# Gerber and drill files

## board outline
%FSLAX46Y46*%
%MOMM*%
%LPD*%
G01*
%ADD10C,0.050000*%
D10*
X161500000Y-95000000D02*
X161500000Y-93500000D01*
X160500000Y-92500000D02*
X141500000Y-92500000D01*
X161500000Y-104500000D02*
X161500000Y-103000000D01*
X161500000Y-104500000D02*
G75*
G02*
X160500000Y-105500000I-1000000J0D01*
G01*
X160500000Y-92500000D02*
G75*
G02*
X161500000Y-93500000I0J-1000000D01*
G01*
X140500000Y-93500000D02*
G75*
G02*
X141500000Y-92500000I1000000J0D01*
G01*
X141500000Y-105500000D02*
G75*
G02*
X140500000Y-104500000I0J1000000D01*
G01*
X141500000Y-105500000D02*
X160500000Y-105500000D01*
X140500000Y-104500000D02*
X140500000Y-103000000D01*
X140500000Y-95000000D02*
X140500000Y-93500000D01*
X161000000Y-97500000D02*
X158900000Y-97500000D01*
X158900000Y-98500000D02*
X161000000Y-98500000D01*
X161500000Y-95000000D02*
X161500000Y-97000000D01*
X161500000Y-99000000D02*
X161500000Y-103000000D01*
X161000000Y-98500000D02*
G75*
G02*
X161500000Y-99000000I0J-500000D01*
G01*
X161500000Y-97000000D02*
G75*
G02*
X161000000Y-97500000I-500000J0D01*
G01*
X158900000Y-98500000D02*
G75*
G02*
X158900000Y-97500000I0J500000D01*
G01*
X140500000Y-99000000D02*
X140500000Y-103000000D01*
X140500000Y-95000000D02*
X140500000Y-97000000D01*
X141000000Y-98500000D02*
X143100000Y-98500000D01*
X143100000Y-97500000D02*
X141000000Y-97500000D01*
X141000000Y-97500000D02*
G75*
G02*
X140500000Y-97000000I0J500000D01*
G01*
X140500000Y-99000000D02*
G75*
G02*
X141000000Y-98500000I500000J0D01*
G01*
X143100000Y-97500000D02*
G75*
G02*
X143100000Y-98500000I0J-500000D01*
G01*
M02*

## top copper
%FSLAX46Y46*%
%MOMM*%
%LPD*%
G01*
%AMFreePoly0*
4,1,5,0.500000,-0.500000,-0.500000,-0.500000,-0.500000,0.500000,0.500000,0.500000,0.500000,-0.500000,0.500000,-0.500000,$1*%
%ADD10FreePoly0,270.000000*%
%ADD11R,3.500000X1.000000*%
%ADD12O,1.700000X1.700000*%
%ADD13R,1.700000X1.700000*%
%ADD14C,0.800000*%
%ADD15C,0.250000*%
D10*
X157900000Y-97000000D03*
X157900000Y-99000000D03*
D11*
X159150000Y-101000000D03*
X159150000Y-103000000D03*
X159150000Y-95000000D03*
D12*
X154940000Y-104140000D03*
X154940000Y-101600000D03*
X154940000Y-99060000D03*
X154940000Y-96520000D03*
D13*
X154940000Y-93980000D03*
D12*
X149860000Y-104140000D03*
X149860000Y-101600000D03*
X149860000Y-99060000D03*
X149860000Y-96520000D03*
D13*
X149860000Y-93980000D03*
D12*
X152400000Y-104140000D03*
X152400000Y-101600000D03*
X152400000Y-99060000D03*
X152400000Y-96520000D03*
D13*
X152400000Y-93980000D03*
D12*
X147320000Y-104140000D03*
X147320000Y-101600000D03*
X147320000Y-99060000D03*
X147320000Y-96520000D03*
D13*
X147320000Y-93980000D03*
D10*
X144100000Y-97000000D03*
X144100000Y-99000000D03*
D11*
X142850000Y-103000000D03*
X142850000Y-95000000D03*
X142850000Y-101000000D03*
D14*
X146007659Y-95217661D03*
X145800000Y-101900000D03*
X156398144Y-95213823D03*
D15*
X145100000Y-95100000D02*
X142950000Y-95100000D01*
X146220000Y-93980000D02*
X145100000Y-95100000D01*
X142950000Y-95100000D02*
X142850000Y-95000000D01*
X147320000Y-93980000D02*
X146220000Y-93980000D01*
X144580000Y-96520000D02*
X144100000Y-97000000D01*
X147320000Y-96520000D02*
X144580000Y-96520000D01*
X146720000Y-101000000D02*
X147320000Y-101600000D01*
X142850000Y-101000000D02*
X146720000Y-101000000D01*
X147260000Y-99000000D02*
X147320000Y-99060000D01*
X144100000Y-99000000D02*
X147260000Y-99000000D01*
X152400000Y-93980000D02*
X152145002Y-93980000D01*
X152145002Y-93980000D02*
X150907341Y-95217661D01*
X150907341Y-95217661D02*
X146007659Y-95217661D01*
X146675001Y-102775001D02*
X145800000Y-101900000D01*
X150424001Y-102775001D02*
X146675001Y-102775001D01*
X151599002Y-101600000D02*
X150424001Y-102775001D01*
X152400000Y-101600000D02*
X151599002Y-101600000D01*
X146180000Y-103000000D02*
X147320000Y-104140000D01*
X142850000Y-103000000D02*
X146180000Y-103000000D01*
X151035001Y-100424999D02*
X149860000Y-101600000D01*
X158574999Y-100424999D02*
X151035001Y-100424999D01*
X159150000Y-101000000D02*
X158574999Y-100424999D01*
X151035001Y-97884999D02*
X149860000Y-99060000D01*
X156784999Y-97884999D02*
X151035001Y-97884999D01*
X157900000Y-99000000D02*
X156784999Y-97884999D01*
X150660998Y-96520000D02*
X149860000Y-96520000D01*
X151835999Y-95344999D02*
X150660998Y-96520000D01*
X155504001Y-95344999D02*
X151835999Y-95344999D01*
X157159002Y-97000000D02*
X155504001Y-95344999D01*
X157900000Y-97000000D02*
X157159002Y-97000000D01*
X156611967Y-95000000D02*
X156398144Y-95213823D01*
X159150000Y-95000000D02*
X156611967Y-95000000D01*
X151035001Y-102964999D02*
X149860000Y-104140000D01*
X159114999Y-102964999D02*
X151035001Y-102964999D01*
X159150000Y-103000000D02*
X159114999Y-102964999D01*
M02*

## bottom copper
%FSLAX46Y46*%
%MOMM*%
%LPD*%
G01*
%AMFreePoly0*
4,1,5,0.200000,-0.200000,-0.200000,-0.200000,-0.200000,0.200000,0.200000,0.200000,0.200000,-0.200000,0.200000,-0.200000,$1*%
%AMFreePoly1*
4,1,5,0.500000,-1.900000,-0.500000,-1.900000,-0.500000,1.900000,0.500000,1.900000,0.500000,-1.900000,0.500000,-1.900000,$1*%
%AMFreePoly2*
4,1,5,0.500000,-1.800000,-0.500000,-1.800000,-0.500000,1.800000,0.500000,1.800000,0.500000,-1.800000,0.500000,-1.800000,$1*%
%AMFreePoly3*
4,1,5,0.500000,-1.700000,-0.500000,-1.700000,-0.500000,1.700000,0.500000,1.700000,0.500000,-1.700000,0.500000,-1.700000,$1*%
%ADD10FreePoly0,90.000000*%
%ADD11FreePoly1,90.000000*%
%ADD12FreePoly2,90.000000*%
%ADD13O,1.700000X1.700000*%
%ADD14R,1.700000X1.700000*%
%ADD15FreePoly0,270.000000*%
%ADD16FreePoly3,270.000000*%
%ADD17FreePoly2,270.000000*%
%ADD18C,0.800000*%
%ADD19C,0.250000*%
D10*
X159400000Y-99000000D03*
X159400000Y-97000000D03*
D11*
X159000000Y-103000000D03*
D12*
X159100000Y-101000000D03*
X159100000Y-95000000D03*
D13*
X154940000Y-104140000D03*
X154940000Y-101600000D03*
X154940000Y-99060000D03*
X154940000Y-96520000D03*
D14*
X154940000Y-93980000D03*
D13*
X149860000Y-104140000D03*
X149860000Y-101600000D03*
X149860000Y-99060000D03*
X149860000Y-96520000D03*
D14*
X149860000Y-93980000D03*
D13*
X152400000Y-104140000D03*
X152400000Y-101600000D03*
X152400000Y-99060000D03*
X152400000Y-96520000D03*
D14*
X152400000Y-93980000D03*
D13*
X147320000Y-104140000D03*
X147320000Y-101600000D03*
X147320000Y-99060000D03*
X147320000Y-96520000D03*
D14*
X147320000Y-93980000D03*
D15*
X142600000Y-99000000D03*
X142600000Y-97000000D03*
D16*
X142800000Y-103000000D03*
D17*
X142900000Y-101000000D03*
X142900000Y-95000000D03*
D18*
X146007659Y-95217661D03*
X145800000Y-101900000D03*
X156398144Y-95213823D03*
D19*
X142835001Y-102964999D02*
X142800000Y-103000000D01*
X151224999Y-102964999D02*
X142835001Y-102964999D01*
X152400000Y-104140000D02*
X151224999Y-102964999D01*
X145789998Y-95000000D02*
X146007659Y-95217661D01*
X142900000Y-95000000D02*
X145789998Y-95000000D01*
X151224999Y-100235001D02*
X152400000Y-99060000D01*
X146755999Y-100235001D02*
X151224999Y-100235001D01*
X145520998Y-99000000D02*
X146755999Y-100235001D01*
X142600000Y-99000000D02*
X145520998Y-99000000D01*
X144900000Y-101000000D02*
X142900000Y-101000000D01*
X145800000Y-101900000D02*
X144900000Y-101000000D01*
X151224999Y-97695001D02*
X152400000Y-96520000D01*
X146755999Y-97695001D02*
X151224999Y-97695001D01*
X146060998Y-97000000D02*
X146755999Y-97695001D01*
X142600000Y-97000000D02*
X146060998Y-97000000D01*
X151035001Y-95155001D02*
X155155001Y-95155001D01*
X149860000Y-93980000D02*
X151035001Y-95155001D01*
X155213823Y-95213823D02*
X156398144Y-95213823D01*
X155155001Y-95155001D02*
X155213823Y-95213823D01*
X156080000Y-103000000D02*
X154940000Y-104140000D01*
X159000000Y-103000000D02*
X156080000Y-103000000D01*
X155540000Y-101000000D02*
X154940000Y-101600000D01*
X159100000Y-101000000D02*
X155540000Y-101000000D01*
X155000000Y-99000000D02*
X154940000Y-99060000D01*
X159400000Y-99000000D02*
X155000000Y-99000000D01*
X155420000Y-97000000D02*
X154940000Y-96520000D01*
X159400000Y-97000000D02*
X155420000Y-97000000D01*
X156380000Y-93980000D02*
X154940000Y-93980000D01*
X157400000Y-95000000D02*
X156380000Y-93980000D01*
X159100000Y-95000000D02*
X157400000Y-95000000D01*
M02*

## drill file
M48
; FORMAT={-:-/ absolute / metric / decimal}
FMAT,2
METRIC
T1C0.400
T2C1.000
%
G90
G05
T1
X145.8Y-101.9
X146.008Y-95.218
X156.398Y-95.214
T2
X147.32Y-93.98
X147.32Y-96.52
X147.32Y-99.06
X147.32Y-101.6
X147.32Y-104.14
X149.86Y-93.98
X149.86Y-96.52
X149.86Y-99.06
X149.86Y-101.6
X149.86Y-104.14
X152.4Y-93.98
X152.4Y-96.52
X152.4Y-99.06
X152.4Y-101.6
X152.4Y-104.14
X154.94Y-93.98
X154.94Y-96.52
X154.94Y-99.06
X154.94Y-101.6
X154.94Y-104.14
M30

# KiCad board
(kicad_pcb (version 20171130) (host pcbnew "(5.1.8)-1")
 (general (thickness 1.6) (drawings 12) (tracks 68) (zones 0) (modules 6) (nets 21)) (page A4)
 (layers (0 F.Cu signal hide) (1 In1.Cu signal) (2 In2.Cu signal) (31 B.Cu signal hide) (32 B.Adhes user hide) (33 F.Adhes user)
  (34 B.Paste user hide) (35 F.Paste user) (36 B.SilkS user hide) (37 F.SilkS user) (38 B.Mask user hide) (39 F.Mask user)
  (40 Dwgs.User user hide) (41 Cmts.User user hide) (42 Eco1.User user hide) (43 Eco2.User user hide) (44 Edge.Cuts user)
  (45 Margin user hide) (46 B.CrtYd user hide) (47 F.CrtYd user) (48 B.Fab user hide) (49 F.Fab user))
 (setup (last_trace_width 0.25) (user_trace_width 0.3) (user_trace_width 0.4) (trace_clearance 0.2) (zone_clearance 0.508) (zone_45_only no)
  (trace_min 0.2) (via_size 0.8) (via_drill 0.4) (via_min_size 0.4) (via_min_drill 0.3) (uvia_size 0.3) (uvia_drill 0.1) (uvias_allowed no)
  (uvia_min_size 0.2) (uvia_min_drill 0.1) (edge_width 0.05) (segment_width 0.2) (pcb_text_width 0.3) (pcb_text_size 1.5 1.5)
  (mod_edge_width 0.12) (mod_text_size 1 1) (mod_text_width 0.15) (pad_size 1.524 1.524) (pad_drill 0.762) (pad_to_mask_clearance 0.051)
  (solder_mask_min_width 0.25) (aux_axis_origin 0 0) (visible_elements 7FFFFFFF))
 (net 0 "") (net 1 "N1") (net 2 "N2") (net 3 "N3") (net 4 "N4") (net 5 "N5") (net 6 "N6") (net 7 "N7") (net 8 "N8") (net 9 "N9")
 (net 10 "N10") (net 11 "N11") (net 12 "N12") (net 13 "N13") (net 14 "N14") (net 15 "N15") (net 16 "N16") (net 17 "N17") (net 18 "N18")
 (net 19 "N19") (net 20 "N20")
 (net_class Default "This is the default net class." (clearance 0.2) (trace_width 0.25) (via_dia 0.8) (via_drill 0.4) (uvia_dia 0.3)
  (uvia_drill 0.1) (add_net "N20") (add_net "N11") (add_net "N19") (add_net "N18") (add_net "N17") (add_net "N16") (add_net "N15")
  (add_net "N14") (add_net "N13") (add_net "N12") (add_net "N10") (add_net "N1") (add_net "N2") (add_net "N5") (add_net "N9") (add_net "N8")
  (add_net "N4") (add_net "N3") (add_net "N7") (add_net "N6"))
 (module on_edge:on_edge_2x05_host (layer F.Cu) (at 161.5 99 270)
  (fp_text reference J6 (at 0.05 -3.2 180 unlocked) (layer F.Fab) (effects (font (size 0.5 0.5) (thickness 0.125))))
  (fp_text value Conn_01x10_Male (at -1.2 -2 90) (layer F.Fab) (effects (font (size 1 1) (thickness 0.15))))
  (fp_line (start -1.5 0.5) (end -1.5 2.6) (layer Edge.Cuts) (width 0.05))
  (fp_line (start -0.5 2.6) (end -0.5 0.5) (layer Edge.Cuts) (width 0.05))
  (fp_line (start -4 0) (end -2 0) (layer Edge.Cuts) (width 0.05))
  (fp_line (start 0 0) (end 4 0) (layer Edge.Cuts) (width 0.05))
  (fp_arc (start 0 0.5) (end 0 0) (angle -90) (layer Edge.Cuts) (width 0.05))
  (fp_arc (start -2 0.5) (end -1.5 0.5) (angle -90) (layer Edge.Cuts) (width 0.05))
  (fp_arc (start -1 2.6) (end -1.5 2.6) (angle -180) (layer Edge.Cuts) (width 0.05))
  (pad 2 smd custom (at -2 3.6 270) (size 1 1) (layers F.Cu F.Mask) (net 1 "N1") (zone_connect 0)
   (options (clearance outline) (anchor rect)) (primitives))
  (pad 3 smd custom (at 0 3.6 270) (size 1 1) (layers F.Cu F.Mask) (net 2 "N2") (zone_connect 0) (options (clearance outline) (anchor rect))
   (primitives))
  (pad 8 smd custom (at 0 2.1 90) (size 0.4 0.4) (layers B.Cu B.Mask) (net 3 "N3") (zone_connect 0)
   (options (clearance outline) (anchor rect)) (primitives))
  (pad 7 smd custom (at -2 2.1 90) (size 0.4 0.4) (layers B.Cu B.Mask) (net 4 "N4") (zone_connect 0)
   (options (clearance outline) (anchor rect)) (primitives))
  (pad 4 smd rect (at 2 2.35 270) (size 1 3.5) (layers F.Cu F.Mask) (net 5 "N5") (zone_connect 0))
  (pad 10 smd custom (at 4 2.5 90) (size 1 3.8) (layers B.Cu B.Mask) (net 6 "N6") (zone_connect 0)
   (options (clearance outline) (anchor rect)) (primitives))
  (pad 9 smd custom (at 2 2.4 90) (size 1 3.6) (layers B.Cu B.Mask) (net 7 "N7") (zone_connect 0)
   (options (clearance outline) (anchor rect)) (primitives))
  (pad 6 smd custom (at -4 2.4 90) (size 1 3.6) (layers B.Cu B.Mask) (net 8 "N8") (zone_connect 0)
   (options (clearance outline) (anchor rect)) (primitives))
  (pad 5 smd rect (at 4 2.35 270) (size 1 3.5) (layers F.Cu F.Mask) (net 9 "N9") (zone_connect 0))
  (pad 1 smd rect (at -4 2.35 270) (size 1 3.5) (layers F.Cu F.Mask) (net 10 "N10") (zone_connect 0)))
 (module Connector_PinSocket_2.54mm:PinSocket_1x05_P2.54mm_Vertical (layer F.Cu) (at 154.94 93.98)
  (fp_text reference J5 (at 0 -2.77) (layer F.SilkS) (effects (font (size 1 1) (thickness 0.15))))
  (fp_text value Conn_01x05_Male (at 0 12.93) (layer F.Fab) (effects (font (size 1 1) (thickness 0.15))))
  (pad 5 thru_hole oval (at 0 10.16) (size 1.7 1.7) (drill 1) (layers *.Cu *.Mask) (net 6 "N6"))
  (pad 4 thru_hole oval (at 0 7.62) (size 1.7 1.7) (drill 1) (layers *.Cu *.Mask) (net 7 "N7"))
  (pad 3 thru_hole oval (at 0 5.08) (size 1.7 1.7) (drill 1) (layers *.Cu *.Mask) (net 3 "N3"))
  (pad 2 thru_hole oval (at 0 2.54) (size 1.7 1.7) (drill 1) (layers *.Cu *.Mask) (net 4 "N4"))
  (pad 1 thru_hole rect (at 0 0) (size 1.7 1.7) (drill 1) (layers *.Cu *.Mask) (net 8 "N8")))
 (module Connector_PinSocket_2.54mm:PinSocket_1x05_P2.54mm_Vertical (layer F.Cu) (at 149.86 93.98)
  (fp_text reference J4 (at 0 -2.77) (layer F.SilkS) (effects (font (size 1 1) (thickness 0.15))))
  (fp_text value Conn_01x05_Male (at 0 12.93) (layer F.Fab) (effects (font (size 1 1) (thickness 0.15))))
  (pad 5 thru_hole oval (at 0 10.16) (size 1.7 1.7) (drill 1) (layers *.Cu *.Mask) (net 9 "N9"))
  (pad 4 thru_hole oval (at 0 7.62) (size 1.7 1.7) (drill 1) (layers *.Cu *.Mask) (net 5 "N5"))
  (pad 3 thru_hole oval (at 0 5.08) (size 1.7 1.7) (drill 1) (layers *.Cu *.Mask) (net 2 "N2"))
  (pad 2 thru_hole oval (at 0 2.54) (size 1.7 1.7) (drill 1) (layers *.Cu *.Mask) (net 1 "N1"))
  (pad 1 thru_hole rect (at 0 0) (size 1.7 1.7) (drill 1) (layers *.Cu *.Mask) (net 10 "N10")))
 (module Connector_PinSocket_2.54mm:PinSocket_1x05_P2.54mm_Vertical (layer F.Cu) (at 152.4 93.98)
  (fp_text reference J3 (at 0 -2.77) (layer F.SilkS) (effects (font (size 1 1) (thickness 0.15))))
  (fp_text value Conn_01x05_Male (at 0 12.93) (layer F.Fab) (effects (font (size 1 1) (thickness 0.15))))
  (pad 5 thru_hole oval (at 0 10.16) (size 1.7 1.7) (drill 1) (layers *.Cu *.Mask) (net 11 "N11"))
  (pad 4 thru_hole oval (at 0 7.62) (size 1.7 1.7) (drill 1) (layers *.Cu *.Mask) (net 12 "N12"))
  (pad 3 thru_hole oval (at 0 5.08) (size 1.7 1.7) (drill 1) (layers *.Cu *.Mask) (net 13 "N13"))
  (pad 2 thru_hole oval (at 0 2.54) (size 1.7 1.7) (drill 1) (layers *.Cu *.Mask) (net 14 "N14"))
  (pad 1 thru_hole rect (at 0 0) (size 1.7 1.7) (drill 1) (layers *.Cu *.Mask) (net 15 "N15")))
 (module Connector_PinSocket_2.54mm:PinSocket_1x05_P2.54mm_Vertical (layer F.Cu) (at 147.32 93.98)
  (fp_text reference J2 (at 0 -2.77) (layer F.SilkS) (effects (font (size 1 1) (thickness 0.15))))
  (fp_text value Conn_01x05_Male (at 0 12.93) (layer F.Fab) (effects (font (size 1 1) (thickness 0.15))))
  (pad 5 thru_hole oval (at 0 10.16) (size 1.7 1.7) (drill 1) (layers *.Cu *.Mask) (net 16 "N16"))
  (pad 4 thru_hole oval (at 0 7.62) (size 1.7 1.7) (drill 1) (layers *.Cu *.Mask) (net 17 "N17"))
  (pad 3 thru_hole oval (at 0 5.08) (size 1.7 1.7) (drill 1) (layers *.Cu *.Mask) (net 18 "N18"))
  (pad 2 thru_hole oval (at 0 2.54) (size 1.7 1.7) (drill 1) (layers *.Cu *.Mask) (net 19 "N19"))
  (pad 1 thru_hole rect (at 0 0) (size 1.7 1.7) (drill 1) (layers *.Cu *.Mask) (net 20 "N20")))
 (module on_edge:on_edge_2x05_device (layer F.Cu) (at 140.5 99 270)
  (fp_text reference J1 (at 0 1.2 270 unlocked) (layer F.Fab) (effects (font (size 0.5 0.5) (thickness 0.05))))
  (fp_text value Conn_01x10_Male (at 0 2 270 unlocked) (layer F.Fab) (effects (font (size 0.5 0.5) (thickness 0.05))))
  (fp_line (start 0 0) (end 4 0) (layer Edge.Cuts) (width 0.05))
  (fp_line (start -4 0) (end -2 0) (layer Edge.Cuts) (width 0.05))
  (fp_line (start -0.5 -0.5) (end -0.5 -2.6) (layer Edge.Cuts) (width 0.05))
  (fp_line (start -1.5 -2.6) (end -1.5 -0.5) (layer Edge.Cuts) (width 0.05))
  (fp_arc (start -2 -0.5) (end -2 0) (angle -90) (layer Edge.Cuts) (width 0.05))
  (fp_arc (start 0 -0.5) (end -0.5 -0.5) (angle -90) (layer Edge.Cuts) (width 0.05))
  (fp_arc (start -1 -2.6) (end -0.5 -2.6) (angle -180) (layer Edge.Cuts) (width 0.05))
  (pad 2 smd custom (at -2 -3.6 270) (size 1 1) (layers F.Cu F.Mask) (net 19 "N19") (zone_connect 0)
   (options (clearance outline) (anchor rect)) (primitives))
  (pad 3 smd custom (at 0 -3.6 270) (size 1 1) (layers F.Cu F.Mask) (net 18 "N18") (zone_connect 0)
   (options (clearance outline) (anchor rect)) (primitives))
  (pad 8 smd custom (at 0 -2.1 270) (size 0.4 0.4) (layers B.Cu B.Mask) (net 13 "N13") (zone_connect 0)
   (options (clearance outline) (anchor rect)) (primitives))
  (pad 7 smd custom (at -2 -2.1 270) (size 0.4 0.4) (layers B.Cu B.Mask) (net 14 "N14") (zone_connect 0)
   (options (clearance outline) (anchor rect)) (primitives))
  (pad 10 smd custom (at 4 -2.3 270) (size 1 3.4) (layers B.Cu B.Mask) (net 11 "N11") (zone_connect 0)
   (options (clearance outline) (anchor rect)) (primitives))
  (pad 9 smd custom (at 2 -2.4 270) (size 1 3.6) (layers B.Cu B.Mask) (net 12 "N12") (zone_connect 0)
   (options (clearance outline) (anchor rect)) (primitives))
  (pad 6 smd custom (at -4 -2.4 270) (size 1 3.6) (layers B.Cu B.Mask) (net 15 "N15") (zone_connect 0)
   (options (clearance outline) (anchor rect)) (primitives))
  (pad 5 smd rect (at 4 -2.35 90) (size 1 3.5) (layers F.Cu F.Mask) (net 16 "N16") (zone_connect 0))
  (pad 1 smd rect (at -4 -2.35 90) (size 1 3.5) (layers F.Cu F.Mask) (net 20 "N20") (zone_connect 0))
  (pad 4 smd rect (at 2 -2.35 90) (size 1 3.5) (layers F.Cu F.Mask) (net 17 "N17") (zone_connect 0)))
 (gr_line (start 161.5 95) (end 161.5 93.5) (layer Edge.Cuts) (width 0.05))
 (gr_line (start 160.5 92.5) (end 141.5 92.5) (layer Edge.Cuts) (width 0.05))
 (gr_line (start 161.5 104.5) (end 161.5 103) (layer Edge.Cuts) (width 0.05))
 (gr_arc (start 160.5 104.5) (end 160.5 105.5) (angle -90) (layer Edge.Cuts) (width 0.05))
 (gr_arc (start 160.5 93.5) (end 161.5 93.5) (angle -90) (layer Edge.Cuts) (width 0.05))
 (gr_arc (start 141.5 93.5) (end 141.5 92.5) (angle -90) (layer Edge.Cuts) (width 0.05))
 (gr_arc (start 141.5 104.5) (end 140.5 104.5) (angle -90) (layer Edge.Cuts) (width 0.05))
 (gr_line (start 141.5 105.5) (end 160.5 105.5) (layer Edge.Cuts) (width 0.05))
 (gr_line (start 140.5 104.5) (end 140.5 103) (layer Edge.Cuts) (width 0.05))
 (gr_line (start 140.5 95) (end 140.5 93.5) (layer Edge.Cuts) (width 0.05))
 (segment (start 145.1 95.1) (end 142.95 95.1) (width 0.25) (layer F.Cu) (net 20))
 (segment (start 146.22 93.98) (end 145.1 95.1) (width 0.25) (layer F.Cu) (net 20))
 (segment (start 142.95 95.1) (end 142.85 95) (width 0.25) (layer F.Cu) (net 20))
 (segment (start 147.32 93.98) (end 146.22 93.98) (width 0.25) (layer F.Cu) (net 20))
 (segment (start 144.58 96.52) (end 144.1 97) (width 0.25) (layer F.Cu) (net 19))
 (segment (start 147.32 96.52) (end 144.58 96.52) (width 0.25) (layer F.Cu) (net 19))
 (segment (start 146.72 101) (end 147.32 101.6) (width 0.25) (layer F.Cu) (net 17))
 (segment (start 142.85 101) (end 146.72 101) (width 0.25) (layer F.Cu) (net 17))
 (segment (start 147.26 99) (end 147.32 99.06) (width 0.25) (layer F.Cu) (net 18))
 (segment (start 144.1 99) (end 147.26 99) (width 0.25) (layer F.Cu) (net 18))
 (segment (start 142.835001 102.964999) (end 142.8 103) (width 0.25) (layer B.Cu) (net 11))
 (segment (start 151.224999 102.964999) (end 142.835001 102.964999) (width 0.25) (layer B.Cu) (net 11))
 (segment (start 152.4 104.14) (end 151.224999 102.964999) (width 0.25) (layer B.Cu) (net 11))
 (segment (start 145.789998 95) (end 146.007659 95.217661) (width 0.25) (layer B.Cu) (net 15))
 (via (at 146.007659 95.217661) (size 0.8) (drill 0.4) (layers F.Cu B.Cu) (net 15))
 (segment (start 152.4 93.98) (end 152.145002 93.98) (width 0.25) (layer F.Cu) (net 15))
 (segment (start 152.145002 93.98) (end 150.907341 95.217661) (width 0.25) (layer F.Cu) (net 15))
 (segment (start 150.907341 95.217661) (end 146.007659 95.217661) (width 0.25) (layer F.Cu) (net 15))
 (segment (start 142.9 95) (end 145.789998 95) (width 0.25) (layer B.Cu) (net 15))
 (segment (start 151.224999 100.235001) (end 152.4 99.06) (width 0.25) (layer B.Cu) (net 13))
 (segment (start 146.755999 100.235001) (end 151.224999 100.235001) (width 0.25) (layer B.Cu) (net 13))
 (segment (start 145.520998 99) (end 146.755999 100.235001) (width 0.25) (layer B.Cu) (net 13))
 (segment (start 142.6 99) (end 145.520998 99) (width 0.25) (layer B.Cu) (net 13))
 (segment (start 146.675001 102.775001) (end 145.8 101.9) (width 0.25) (layer F.Cu) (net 12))
 (segment (start 150.424001 102.775001) (end 146.675001 102.775001) (width 0.25) (layer F.Cu) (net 12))
 (via (at 145.8 101.9) (size 0.8) (drill 0.4) (layers F.Cu B.Cu) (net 12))
 (segment (start 151.599002 101.6) (end 150.424001 102.775001) (width 0.25) (layer F.Cu) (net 12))
 (segment (start 152.4 101.6) (end 151.599002 101.6) (width 0.25) (layer F.Cu) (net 12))
 (segment (start 144.9 101) (end 142.9 101) (width 0.25) (layer B.Cu) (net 12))
 (segment (start 145.8 101.9) (end 144.9 101) (width 0.25) (layer B.Cu) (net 12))
 (segment (start 151.224999 97.695001) (end 152.4 96.52) (width 0.25) (layer B.Cu) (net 14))
 (segment (start 146.755999 97.695001) (end 151.224999 97.695001) (width 0.25) (layer B.Cu) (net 14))
 (segment (start 146.060998 97) (end 146.755999 97.695001) (width 0.25) (layer B.Cu) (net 14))
 (segment (start 142.6 97) (end 146.060998 97) (width 0.25) (layer B.Cu) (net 14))
 (segment (start 146.18 103) (end 147.32 104.14) (width 0.25) (layer F.Cu) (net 16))
 (segment (start 142.85 103) (end 146.18 103) (width 0.25) (layer F.Cu) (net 16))
 (segment (start 151.035001 100.424999) (end 149.86 101.6) (width 0.25) (layer F.Cu) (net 5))
 (segment (start 158.574999 100.424999) (end 151.035001 100.424999) (width 0.25) (layer F.Cu) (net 5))
 (segment (start 159.15 101) (end 158.574999 100.424999) (width 0.25) (layer F.Cu) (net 5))
 (segment (start 151.035001 97.884999) (end 149.86 99.06) (width 0.25) (layer F.Cu) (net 2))
 (segment (start 156.784999 97.884999) (end 151.035001 97.884999) (width 0.25) (layer F.Cu) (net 2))
 (segment (start 157.9 99) (end 156.784999 97.884999) (width 0.25) (layer F.Cu) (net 2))
 (segment (start 150.660998 96.52) (end 149.86 96.52) (width 0.25) (layer F.Cu) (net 1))
 (segment (start 151.835999 95.344999) (end 150.660998 96.52) (width 0.25) (layer F.Cu) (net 1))
 (segment (start 155.504001 95.344999) (end 151.835999 95.344999) (width 0.25) (layer F.Cu) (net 1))
 (segment (start 157.159002 97) (end 155.504001 95.344999) (width 0.25) (layer F.Cu) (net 1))
 (segment (start 157.9 97) (end 157.159002 97) (width 0.25) (layer F.Cu) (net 1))
 (segment (start 151.035001 95.155001) (end 155.155001 95.155001) (width 0.25) (layer B.Cu) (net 10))
 (segment (start 149.86 93.98) (end 151.035001 95.155001) (width 0.25) (layer B.Cu) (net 10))
 (segment (start 155.213823 95.213823) (end 156.398144 95.213823) (width 0.25) (layer B.Cu) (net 10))
 (segment (start 155.155001 95.155001) (end 155.213823 95.213823) (width 0.25) (layer B.Cu) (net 10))
 (via (at 156.398144 95.213823) (size 0.8) (drill 0.4) (layers F.Cu B.Cu) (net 10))
 (segment (start 156.611967 95) (end 156.398144 95.213823) (width 0.25) (layer F.Cu) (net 10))
 (segment (start 159.15 95) (end 156.611967 95) (width 0.25) (layer F.Cu) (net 10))
 (segment (start 151.035001 102.964999) (end 149.86 104.14) (width 0.25) (layer F.Cu) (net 9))
 (segment (start 159.114999 102.964999) (end 151.035001 102.964999) (width 0.25) (layer F.Cu) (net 9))
 (segment (start 159.15 103) (end 159.114999 102.964999) (width 0.25) (layer F.Cu) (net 9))
 (segment (start 156.08 103) (end 154.94 104.14) (width 0.25) (layer B.Cu) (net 6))
 (segment (start 159 103) (end 156.08 103) (width 0.25) (layer B.Cu) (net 6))
 (segment (start 155.54 101) (end 154.94 101.6) (width 0.25) (layer B.Cu) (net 7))
 (segment (start 159.1 101) (end 155.54 101) (width 0.25) (layer B.Cu) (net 7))
 (segment (start 155 99) (end 154.94 99.06) (width 0.25) (layer B.Cu) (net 3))
 (segment (start 159.4 99) (end 155 99) (width 0.25) (layer B.Cu) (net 3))
 (segment (start 155.42 97) (end 154.94 96.52) (width 0.25) (layer B.Cu) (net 4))
 (segment (start 159.4 97) (end 155.42 97) (width 0.25) (layer B.Cu) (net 4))
 (segment (start 156.38 93.98) (end 154.94 93.98) (width 0.25) (layer B.Cu) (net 8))
 (segment (start 157.4 95) (end 156.38 93.98) (width 0.25) (layer B.Cu) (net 8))
 (segment (start 159.1 95) (end 157.4 95) (width 0.25) (layer B.Cu) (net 8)))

